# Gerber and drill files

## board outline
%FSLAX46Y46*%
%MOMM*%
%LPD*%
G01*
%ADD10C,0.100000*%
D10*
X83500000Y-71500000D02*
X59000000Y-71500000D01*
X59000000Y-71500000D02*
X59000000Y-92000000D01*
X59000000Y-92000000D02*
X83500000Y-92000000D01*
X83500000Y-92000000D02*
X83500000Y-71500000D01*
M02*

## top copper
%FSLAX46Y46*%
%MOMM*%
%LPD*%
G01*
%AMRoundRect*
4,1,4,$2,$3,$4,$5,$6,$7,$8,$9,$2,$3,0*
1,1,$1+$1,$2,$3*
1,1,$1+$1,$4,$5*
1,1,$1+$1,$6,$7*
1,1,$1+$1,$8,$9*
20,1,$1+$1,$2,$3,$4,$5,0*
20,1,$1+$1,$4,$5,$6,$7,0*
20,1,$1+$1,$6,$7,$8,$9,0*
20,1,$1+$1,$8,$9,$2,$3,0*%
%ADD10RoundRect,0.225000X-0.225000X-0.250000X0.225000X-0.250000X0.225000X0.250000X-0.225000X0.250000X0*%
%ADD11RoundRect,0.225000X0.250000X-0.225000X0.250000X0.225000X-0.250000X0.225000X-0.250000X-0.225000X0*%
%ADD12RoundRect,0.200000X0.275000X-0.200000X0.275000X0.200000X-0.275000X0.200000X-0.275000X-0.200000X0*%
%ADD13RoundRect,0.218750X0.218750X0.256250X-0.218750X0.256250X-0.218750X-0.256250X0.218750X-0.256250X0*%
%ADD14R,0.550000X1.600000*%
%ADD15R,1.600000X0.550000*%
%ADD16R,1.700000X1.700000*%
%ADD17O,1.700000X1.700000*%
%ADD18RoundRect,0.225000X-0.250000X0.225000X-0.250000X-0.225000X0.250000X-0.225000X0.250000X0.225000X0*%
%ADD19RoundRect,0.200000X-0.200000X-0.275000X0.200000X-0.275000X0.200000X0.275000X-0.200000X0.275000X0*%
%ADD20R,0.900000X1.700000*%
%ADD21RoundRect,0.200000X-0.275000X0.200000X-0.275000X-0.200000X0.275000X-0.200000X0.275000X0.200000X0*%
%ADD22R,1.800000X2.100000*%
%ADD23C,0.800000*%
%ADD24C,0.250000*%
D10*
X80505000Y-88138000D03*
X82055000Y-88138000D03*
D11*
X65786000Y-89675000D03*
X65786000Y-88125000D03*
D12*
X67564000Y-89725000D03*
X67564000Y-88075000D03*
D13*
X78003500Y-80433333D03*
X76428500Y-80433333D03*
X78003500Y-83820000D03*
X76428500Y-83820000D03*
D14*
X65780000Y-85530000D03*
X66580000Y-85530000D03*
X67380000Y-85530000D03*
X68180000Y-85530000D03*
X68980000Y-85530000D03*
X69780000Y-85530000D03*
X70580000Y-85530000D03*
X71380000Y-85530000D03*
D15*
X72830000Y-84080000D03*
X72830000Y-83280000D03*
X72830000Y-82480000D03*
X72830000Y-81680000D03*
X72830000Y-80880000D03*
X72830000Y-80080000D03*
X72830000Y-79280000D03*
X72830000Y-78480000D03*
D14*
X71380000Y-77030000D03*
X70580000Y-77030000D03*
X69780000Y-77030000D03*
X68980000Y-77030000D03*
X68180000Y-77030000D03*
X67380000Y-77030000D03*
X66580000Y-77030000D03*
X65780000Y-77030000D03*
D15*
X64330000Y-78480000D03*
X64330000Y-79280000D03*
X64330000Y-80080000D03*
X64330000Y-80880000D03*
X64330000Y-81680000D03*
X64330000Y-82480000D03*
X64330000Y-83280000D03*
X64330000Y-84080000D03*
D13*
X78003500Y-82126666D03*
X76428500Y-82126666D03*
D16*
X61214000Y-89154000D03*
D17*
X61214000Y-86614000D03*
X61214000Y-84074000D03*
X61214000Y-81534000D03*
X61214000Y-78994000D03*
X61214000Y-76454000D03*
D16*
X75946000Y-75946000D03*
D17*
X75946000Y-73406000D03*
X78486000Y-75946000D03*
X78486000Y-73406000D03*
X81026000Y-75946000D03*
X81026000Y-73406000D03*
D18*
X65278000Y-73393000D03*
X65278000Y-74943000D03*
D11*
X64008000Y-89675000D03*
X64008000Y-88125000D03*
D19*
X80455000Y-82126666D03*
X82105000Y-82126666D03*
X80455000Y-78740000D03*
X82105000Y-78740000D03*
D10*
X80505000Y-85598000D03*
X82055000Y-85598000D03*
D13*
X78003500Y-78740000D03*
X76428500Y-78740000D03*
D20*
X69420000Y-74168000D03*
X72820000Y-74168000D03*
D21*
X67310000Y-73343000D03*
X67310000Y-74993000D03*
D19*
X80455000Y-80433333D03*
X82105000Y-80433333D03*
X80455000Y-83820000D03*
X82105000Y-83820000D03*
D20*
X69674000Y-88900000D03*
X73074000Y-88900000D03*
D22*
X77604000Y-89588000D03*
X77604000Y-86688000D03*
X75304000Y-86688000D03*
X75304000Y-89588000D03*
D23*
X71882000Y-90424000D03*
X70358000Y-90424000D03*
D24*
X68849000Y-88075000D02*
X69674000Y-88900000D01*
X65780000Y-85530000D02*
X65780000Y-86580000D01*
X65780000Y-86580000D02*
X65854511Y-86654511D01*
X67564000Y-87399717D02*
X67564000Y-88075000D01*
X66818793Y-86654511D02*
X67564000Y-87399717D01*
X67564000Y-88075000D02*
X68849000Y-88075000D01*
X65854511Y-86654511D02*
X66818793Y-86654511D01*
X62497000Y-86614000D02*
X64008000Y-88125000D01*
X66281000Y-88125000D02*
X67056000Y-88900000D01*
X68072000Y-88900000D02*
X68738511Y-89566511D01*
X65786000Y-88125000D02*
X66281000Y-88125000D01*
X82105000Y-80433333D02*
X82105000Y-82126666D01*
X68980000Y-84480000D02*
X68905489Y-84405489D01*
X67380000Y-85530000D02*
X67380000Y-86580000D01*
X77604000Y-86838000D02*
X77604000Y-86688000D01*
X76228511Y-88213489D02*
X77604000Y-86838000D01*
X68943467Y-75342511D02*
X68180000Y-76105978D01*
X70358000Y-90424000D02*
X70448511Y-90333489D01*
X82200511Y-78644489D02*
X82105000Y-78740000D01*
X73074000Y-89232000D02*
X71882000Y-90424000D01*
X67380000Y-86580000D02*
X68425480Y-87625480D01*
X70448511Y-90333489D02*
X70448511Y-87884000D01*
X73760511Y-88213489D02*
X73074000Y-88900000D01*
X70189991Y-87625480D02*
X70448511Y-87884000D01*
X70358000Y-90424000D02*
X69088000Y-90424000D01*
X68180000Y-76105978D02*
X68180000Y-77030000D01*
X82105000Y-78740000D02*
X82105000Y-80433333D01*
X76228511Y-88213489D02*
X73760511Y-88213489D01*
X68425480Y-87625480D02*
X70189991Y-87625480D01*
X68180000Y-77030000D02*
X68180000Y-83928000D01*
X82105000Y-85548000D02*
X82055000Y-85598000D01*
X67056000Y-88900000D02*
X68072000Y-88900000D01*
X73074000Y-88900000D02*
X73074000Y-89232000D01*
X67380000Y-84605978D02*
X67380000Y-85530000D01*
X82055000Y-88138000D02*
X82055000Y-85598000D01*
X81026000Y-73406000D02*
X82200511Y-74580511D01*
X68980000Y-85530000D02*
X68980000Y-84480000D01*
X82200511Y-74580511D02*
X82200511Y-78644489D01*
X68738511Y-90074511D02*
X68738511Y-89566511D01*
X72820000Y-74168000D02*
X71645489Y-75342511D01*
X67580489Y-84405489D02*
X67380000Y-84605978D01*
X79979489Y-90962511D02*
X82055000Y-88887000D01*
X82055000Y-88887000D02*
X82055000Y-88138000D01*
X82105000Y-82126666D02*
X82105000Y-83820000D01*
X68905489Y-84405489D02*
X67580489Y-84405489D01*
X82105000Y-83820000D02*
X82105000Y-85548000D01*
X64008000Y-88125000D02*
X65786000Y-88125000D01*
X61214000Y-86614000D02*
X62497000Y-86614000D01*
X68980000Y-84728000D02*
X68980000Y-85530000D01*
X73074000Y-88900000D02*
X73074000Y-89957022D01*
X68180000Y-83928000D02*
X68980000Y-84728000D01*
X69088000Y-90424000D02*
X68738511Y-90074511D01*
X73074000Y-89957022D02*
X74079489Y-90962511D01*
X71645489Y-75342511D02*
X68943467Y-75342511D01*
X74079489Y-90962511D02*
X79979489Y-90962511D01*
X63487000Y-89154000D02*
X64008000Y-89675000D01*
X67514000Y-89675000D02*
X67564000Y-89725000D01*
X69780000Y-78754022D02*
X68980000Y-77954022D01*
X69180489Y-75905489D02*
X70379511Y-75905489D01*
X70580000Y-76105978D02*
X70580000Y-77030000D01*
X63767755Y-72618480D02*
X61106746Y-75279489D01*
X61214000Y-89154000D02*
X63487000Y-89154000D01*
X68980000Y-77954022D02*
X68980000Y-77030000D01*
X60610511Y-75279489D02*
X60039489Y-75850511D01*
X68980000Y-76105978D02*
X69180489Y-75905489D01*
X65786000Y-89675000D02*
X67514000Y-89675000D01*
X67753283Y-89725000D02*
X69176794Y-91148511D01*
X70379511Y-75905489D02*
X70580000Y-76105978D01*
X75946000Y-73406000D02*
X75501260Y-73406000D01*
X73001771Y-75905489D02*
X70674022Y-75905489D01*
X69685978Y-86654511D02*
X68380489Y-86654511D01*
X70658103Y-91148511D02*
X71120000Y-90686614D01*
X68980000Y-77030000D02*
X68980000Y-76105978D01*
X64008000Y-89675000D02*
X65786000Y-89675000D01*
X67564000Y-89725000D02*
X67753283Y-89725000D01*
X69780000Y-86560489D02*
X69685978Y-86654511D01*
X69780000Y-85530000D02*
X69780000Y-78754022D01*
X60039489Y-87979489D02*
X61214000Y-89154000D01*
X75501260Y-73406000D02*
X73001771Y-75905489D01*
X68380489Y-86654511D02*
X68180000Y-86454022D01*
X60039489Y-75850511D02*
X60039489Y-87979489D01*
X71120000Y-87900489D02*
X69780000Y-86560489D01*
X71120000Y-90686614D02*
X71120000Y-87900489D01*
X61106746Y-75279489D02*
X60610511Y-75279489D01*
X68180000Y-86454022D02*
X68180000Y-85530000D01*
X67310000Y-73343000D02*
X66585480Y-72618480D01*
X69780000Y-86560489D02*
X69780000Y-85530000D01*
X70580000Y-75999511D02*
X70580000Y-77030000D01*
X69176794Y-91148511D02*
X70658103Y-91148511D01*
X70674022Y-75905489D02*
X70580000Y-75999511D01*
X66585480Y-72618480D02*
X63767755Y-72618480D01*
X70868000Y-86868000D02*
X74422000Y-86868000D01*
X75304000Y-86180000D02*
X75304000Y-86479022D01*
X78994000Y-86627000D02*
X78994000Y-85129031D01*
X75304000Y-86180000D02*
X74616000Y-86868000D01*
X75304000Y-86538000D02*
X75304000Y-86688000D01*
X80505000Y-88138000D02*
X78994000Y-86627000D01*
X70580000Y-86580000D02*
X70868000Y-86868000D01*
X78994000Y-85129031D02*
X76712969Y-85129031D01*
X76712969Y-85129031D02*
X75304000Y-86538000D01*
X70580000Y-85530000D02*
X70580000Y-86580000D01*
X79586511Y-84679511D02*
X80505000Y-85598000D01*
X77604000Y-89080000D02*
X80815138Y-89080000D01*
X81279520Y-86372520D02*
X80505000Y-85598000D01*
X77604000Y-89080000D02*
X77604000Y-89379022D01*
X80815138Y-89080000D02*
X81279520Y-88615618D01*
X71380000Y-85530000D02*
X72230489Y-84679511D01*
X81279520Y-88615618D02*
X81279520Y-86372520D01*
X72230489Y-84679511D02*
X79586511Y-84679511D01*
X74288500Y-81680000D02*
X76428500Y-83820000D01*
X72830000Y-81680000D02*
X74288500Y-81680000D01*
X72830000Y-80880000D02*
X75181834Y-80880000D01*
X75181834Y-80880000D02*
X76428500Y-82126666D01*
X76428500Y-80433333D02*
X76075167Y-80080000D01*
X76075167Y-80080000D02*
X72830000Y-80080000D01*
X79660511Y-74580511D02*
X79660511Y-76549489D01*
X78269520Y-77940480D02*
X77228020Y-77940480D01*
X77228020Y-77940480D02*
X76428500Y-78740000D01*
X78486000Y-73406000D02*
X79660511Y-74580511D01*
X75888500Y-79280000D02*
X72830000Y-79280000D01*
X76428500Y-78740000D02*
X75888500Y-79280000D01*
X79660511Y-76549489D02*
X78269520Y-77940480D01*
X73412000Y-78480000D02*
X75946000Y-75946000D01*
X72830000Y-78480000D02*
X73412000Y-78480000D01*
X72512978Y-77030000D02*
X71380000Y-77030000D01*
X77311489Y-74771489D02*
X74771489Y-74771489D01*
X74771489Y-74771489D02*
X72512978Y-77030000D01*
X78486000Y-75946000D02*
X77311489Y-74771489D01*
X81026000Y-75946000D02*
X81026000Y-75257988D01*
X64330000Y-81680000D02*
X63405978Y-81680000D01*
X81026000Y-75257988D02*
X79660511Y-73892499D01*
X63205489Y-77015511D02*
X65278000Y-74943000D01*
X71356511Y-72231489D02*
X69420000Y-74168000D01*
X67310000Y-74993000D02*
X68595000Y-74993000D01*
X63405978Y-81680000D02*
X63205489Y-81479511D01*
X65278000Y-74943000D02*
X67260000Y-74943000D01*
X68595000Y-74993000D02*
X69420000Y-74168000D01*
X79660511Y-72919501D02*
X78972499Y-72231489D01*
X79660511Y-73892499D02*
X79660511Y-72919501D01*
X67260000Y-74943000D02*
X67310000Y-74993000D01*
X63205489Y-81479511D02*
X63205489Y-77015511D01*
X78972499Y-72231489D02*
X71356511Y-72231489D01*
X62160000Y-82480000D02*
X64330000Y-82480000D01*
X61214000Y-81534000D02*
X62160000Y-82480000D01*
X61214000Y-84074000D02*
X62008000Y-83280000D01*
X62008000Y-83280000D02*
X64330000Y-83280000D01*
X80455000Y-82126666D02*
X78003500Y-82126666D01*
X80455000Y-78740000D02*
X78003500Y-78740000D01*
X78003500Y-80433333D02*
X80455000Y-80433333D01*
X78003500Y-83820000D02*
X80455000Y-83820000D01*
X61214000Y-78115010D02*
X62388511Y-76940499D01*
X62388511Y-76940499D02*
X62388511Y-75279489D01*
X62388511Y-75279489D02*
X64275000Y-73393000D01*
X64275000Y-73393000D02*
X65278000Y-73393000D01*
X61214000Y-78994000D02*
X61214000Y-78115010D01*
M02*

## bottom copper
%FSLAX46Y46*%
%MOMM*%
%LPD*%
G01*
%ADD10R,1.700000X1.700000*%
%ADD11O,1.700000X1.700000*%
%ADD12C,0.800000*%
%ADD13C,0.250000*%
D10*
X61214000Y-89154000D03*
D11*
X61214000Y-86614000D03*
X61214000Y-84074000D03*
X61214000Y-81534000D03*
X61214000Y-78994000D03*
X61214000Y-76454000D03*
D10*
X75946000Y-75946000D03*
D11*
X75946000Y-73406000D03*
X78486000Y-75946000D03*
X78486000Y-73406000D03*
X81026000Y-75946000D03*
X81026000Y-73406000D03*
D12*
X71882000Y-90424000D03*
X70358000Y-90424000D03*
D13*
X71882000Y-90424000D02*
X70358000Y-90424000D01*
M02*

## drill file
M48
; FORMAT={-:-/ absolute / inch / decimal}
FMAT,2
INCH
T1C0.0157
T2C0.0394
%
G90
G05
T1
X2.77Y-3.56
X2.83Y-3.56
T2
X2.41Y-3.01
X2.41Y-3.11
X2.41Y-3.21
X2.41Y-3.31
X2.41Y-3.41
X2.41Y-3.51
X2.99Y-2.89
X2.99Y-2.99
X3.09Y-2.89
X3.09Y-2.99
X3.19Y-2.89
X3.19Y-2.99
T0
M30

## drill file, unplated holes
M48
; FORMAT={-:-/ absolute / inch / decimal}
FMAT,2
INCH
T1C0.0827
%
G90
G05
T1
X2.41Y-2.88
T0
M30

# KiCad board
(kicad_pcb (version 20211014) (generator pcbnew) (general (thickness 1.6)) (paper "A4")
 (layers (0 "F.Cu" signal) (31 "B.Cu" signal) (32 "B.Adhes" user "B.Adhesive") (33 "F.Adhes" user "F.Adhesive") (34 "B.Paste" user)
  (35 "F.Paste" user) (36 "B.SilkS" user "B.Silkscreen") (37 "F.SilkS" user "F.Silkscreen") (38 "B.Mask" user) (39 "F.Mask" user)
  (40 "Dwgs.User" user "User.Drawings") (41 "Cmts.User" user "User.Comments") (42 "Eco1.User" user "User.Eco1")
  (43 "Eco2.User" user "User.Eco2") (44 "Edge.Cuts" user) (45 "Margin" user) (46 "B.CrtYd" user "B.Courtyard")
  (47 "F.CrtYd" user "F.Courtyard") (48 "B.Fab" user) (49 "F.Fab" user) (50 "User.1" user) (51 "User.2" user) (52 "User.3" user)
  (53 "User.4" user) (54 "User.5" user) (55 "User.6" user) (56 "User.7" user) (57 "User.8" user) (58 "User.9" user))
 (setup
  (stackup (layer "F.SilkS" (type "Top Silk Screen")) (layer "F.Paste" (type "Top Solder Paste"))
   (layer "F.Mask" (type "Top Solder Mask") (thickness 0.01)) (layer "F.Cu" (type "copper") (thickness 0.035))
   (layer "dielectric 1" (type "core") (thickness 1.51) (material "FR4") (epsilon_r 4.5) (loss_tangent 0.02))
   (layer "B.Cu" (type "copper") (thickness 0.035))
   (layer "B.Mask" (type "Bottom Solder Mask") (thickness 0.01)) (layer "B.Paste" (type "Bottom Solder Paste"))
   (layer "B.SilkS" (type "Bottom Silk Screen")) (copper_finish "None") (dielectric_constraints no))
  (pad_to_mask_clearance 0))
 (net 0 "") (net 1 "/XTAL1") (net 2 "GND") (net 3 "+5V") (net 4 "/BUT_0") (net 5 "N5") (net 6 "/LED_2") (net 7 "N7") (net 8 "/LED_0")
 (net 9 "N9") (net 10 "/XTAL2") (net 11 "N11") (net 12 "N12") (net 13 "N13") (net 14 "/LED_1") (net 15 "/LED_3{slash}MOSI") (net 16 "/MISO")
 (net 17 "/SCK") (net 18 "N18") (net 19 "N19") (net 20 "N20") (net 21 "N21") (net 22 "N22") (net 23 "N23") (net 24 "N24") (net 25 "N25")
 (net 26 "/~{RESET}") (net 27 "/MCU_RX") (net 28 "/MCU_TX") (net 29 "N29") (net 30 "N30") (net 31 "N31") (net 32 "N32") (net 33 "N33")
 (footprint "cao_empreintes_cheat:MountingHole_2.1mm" (layer "F.Cu") (at 61.214 73.152)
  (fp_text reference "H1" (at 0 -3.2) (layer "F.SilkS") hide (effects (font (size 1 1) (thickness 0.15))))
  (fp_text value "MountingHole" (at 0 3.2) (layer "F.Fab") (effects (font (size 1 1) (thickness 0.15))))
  (pad "" np_thru_hole circle (at 0 0) (size 2.1 2.1) (drill 2.1) (layers *.Cu *.Mask)))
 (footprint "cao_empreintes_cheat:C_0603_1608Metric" (layer "F.Cu") (at 81.28 88.138)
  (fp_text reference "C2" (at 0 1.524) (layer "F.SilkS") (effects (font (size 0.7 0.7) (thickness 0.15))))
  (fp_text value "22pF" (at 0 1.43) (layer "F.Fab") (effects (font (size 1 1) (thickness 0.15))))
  (pad "1" smd roundrect (at -0.775 0) (size 0.9 0.95) (layers "F.Cu" "F.Paste" "F.Mask") (roundrect_rratio 0.25) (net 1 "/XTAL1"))
  (pad "2" smd roundrect (at 0.775 0) (size 0.9 0.95) (layers "F.Cu" "F.Paste" "F.Mask") (roundrect_rratio 0.25) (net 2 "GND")))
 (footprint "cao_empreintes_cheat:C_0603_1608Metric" (layer "F.Cu") (at 65.786 88.9 90)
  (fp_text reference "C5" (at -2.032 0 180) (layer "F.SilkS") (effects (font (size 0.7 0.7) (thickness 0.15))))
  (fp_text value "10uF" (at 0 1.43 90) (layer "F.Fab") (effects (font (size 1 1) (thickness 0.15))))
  (pad "1" smd roundrect (at -0.775 0 90) (size 0.9 0.95) (layers "F.Cu" "F.Paste" "F.Mask") (roundrect_rratio 0.25) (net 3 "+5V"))
  (pad "2" smd roundrect (at 0.775 0 90) (size 0.9 0.95) (layers "F.Cu" "F.Paste" "F.Mask") (roundrect_rratio 0.25) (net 2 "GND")))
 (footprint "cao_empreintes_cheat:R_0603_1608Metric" (layer "F.Cu") (at 67.564 88.9 90)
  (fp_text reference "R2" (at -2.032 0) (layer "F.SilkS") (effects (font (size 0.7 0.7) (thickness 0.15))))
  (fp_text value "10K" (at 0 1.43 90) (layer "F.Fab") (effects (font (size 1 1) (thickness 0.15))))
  (pad "1" smd roundrect (at -0.825 0 90) (size 0.8 0.95) (layers "F.Cu" "F.Paste" "F.Mask") (roundrect_rratio 0.25) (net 3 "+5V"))
  (pad "2" smd roundrect (at 0.825 0 90) (size 0.8 0.95) (layers "F.Cu" "F.Paste" "F.Mask") (roundrect_rratio 0.25) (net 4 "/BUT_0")))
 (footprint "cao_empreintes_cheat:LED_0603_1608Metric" (layer "F.Cu") (at 77.216 80.433333 180)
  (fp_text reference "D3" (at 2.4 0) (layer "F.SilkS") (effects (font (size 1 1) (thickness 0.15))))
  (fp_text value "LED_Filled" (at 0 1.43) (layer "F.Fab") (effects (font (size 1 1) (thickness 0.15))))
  (pad "1" smd roundrect (at -0.7875 0 180) (size 0.875 0.95) (layers "F.Cu" "F.Paste" "F.Mask") (roundrect_rratio 0.25) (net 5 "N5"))
  (pad "2" smd roundrect (at 0.7875 0 180) (size 0.875 0.95) (layers "F.Cu" "F.Paste" "F.Mask") (roundrect_rratio 0.25) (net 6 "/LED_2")))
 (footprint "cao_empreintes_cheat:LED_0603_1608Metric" (layer "F.Cu") (at 77.216 83.82 180)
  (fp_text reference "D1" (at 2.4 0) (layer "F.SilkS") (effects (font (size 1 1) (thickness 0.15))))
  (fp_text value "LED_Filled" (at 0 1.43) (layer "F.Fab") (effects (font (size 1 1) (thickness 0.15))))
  (pad "1" smd roundrect (at -0.7875 0 180) (size 0.875 0.95) (layers "F.Cu" "F.Paste" "F.Mask") (roundrect_rratio 0.25) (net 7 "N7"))
  (pad "2" smd roundrect (at 0.7875 0 180) (size 0.875 0.95) (layers "F.Cu" "F.Paste" "F.Mask") (roundrect_rratio 0.25) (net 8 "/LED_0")))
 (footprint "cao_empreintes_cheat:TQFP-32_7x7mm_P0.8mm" (layer "F.Cu") (at 68.58 81.28 90)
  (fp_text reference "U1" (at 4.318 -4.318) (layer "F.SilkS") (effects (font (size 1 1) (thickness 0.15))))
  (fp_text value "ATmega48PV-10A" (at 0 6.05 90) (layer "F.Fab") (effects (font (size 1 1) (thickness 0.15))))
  (pad "1" smd rect (at -4.25 -2.8 90) (size 1.6 0.55) (layers "F.Cu" "F.Paste" "F.Mask") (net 4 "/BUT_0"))
  (pad "2" smd rect (at -4.25 -2 90) (size 1.6 0.55) (layers "F.Cu" "F.Paste" "F.Mask") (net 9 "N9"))
  (pad "3" smd rect (at -4.25 -1.2 90) (size 1.6 0.55) (layers "F.Cu" "F.Paste" "F.Mask") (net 2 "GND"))
  (pad "4" smd rect (at -4.25 -0.4 90) (size 1.6 0.55) (layers "F.Cu" "F.Paste" "F.Mask") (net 3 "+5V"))
  (pad "5" smd rect (at -4.25 0.4 90) (size 1.6 0.55) (layers "F.Cu" "F.Paste" "F.Mask") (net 2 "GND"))
  (pad "6" smd rect (at -4.25 1.2 90) (size 1.6 0.55) (layers "F.Cu" "F.Paste" "F.Mask") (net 3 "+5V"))
  (pad "7" smd rect (at -4.25 2 90) (size 1.6 0.55) (layers "F.Cu" "F.Paste" "F.Mask") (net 1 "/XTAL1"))
  (pad "8" smd rect (at -4.25 2.8 90) (size 1.6 0.55) (layers "F.Cu" "F.Paste" "F.Mask") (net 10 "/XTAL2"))
  (pad "9" smd rect (at -2.8 4.25 180) (size 1.6 0.55) (layers "F.Cu" "F.Paste" "F.Mask") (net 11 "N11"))
  (pad "10" smd rect (at -2 4.25 180) (size 1.6 0.55) (layers "F.Cu" "F.Paste" "F.Mask") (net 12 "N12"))
  (pad "11" smd rect (at -1.2 4.25 180) (size 1.6 0.55) (layers "F.Cu" "F.Paste" "F.Mask") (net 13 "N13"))
  (pad "12" smd rect (at -0.4 4.25 180) (size 1.6 0.55) (layers "F.Cu" "F.Paste" "F.Mask") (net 8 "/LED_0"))
  (pad "13" smd rect (at 0.4 4.25 180) (size 1.6 0.55) (layers "F.Cu" "F.Paste" "F.Mask") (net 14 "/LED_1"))
  (pad "14" smd rect (at 1.2 4.25 180) (size 1.6 0.55) (layers "F.Cu" "F.Paste" "F.Mask") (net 6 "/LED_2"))
  (pad "15" smd rect (at 2 4.25 180) (size 1.6 0.55) (layers "F.Cu" "F.Paste" "F.Mask") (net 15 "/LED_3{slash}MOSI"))
  (pad "16" smd rect (at 2.8 4.25 180) (size 1.6 0.55) (layers "F.Cu" "F.Paste" "F.Mask") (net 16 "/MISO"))
  (pad "17" smd rect (at 4.25 2.8 90) (size 1.6 0.55) (layers "F.Cu" "F.Paste" "F.Mask") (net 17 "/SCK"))
  (pad "18" smd rect (at 4.25 2 90) (size 1.6 0.55) (layers "F.Cu" "F.Paste" "F.Mask") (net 3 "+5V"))
  (pad "19" smd rect (at 4.25 1.2 90) (size 1.6 0.55) (layers "F.Cu" "F.Paste" "F.Mask") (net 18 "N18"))
  (pad "20" smd rect (at 4.25 0.4 90) (size 1.6 0.55) (layers "F.Cu" "F.Paste" "F.Mask") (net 3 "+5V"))
  (pad "21" smd rect (at 4.25 -0.4 90) (size 1.6 0.55) (layers "F.Cu" "F.Paste" "F.Mask") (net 2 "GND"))
  (pad "22" smd rect (at 4.25 -1.2 90) (size 1.6 0.55) (layers "F.Cu" "F.Paste" "F.Mask") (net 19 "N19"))
  (pad "23" smd rect (at 4.25 -2 90) (size 1.6 0.55) (layers "F.Cu" "F.Paste" "F.Mask") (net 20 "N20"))
  (pad "24" smd rect (at 4.25 -2.8 90) (size 1.6 0.55) (layers "F.Cu" "F.Paste" "F.Mask") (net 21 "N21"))
  (pad "25" smd rect (at 2.8 -4.25 180) (size 1.6 0.55) (layers "F.Cu" "F.Paste" "F.Mask") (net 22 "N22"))
  (pad "26" smd rect (at 2 -4.25 180) (size 1.6 0.55) (layers "F.Cu" "F.Paste" "F.Mask") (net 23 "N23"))
  (pad "27" smd rect (at 1.2 -4.25 180) (size 1.6 0.55) (layers "F.Cu" "F.Paste" "F.Mask") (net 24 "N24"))
  (pad "28" smd rect (at 0.4 -4.25 180) (size 1.6 0.55) (layers "F.Cu" "F.Paste" "F.Mask") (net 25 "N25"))
  (pad "29" smd rect (at -0.4 -4.25 180) (size 1.6 0.55) (layers "F.Cu" "F.Paste" "F.Mask") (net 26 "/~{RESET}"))
  (pad "30" smd rect (at -1.2 -4.25 180) (size 1.6 0.55) (layers "F.Cu" "F.Paste" "F.Mask") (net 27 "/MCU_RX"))
  (pad "31" smd rect (at -2 -4.25 180) (size 1.6 0.55) (layers "F.Cu" "F.Paste" "F.Mask") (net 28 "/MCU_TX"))
  (pad "32" smd rect (at -2.8 -4.25 180) (size 1.6 0.55) (layers "F.Cu" "F.Paste" "F.Mask") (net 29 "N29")))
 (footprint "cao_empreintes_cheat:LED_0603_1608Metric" (layer "F.Cu") (at 77.216 82.126666 180)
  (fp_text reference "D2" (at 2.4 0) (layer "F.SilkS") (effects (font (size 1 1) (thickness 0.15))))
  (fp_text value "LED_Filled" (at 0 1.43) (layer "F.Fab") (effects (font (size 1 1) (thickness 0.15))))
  (pad "1" smd roundrect (at -0.7875 0 180) (size 0.875 0.95) (layers "F.Cu" "F.Paste" "F.Mask") (roundrect_rratio 0.25) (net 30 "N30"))
  (pad "2" smd roundrect (at 0.7875 0 180) (size 0.875 0.95) (layers "F.Cu" "F.Paste" "F.Mask") (roundrect_rratio 0.25) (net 14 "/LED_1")))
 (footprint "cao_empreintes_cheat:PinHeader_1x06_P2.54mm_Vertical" (layer "F.Cu") (at 61.214 89.154 180)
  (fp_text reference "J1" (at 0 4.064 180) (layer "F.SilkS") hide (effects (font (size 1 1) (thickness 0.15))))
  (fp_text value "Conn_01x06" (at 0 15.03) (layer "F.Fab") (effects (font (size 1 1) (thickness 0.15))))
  (pad "1" thru_hole rect (at 0 0 180) (size 1.7 1.7) (drill 1) (layers *.Cu *.Mask) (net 3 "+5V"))
  (pad "2" thru_hole oval (at 0 2.54 180) (size 1.7 1.7) (drill 1) (layers *.Cu *.Mask) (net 2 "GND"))
  (pad "3" thru_hole oval (at 0 5.08 180) (size 1.7 1.7) (drill 1) (layers *.Cu *.Mask) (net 28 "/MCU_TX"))
  (pad "4" thru_hole oval (at 0 7.62 180) (size 1.7 1.7) (drill 1) (layers *.Cu *.Mask) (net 27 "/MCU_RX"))
  (pad "5" thru_hole oval (at 0 10.16 180) (size 1.7 1.7) (drill 1) (layers *.Cu *.Mask) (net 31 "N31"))
  (pad "6" thru_hole oval (at 0 12.7 180) (size 1.7 1.7) (drill 1) (layers *.Cu *.Mask) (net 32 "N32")))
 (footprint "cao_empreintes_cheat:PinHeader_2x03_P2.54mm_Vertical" (layer "F.Cu") (at 75.946 75.946 90)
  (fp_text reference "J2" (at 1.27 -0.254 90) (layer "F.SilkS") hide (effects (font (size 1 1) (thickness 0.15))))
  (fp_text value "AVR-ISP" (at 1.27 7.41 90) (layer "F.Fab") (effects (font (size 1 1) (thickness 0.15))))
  (pad "1" thru_hole rect (at 0 0 90) (size 1.7 1.7) (drill 1) (layers *.Cu *.Mask) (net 16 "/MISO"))
  (pad "2" thru_hole oval (at 2.54 0 90) (size 1.7 1.7) (drill 1) (layers *.Cu *.Mask) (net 3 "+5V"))
  (pad "3" thru_hole oval (at 0 2.54 90) (size 1.7 1.7) (drill 1) (layers *.Cu *.Mask) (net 17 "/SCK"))
  (pad "4" thru_hole oval (at 2.54 2.54 90) (size 1.7 1.7) (drill 1) (layers *.Cu *.Mask) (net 15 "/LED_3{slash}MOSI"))
  (pad "5" thru_hole oval (at 0 5.08 90) (size 1.7 1.7) (drill 1) (layers *.Cu *.Mask) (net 26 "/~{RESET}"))
  (pad "6" thru_hole oval (at 2.54 5.08 90) (size 1.7 1.7) (drill 1) (layers *.Cu *.Mask) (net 2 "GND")))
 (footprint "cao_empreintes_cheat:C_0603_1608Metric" (layer "F.Cu") (at 65.278 74.168 -90)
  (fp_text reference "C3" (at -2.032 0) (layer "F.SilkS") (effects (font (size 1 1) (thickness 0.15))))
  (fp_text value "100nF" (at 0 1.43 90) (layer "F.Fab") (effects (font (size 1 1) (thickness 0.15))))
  (pad "1" smd roundrect (at -0.775 0 270) (size 0.9 0.95) (layers "F.Cu" "F.Paste" "F.Mask") (roundrect_rratio 0.25) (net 31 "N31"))
  (pad "2" smd roundrect (at 0.775 0 270) (size 0.9 0.95) (layers "F.Cu" "F.Paste" "F.Mask") (roundrect_rratio 0.25) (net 26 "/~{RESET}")))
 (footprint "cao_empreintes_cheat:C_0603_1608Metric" (layer "F.Cu") (at 64.008 88.9 90)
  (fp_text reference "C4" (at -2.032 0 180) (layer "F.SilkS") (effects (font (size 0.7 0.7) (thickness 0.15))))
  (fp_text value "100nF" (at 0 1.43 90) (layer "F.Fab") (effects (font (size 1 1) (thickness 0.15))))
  (pad "1" smd roundrect (at -0.775 0 90) (size 0.9 0.95) (layers "F.Cu" "F.Paste" "F.Mask") (roundrect_rratio 0.25) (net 3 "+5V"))
  (pad "2" smd roundrect (at 0.775 0 90) (size 0.9 0.95) (layers "F.Cu" "F.Paste" "F.Mask") (roundrect_rratio 0.25) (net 2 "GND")))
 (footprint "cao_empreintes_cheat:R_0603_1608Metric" (layer "F.Cu") (at 81.28 82.126666)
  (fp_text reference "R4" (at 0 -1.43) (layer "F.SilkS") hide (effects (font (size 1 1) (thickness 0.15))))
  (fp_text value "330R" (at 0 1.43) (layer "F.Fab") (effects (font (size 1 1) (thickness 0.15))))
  (pad "1" smd roundrect (at -0.825 0) (size 0.8 0.95) (layers "F.Cu" "F.Paste" "F.Mask") (roundrect_rratio 0.25) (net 30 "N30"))
  (pad "2" smd roundrect (at 0.825 0) (size 0.8 0.95) (layers "F.Cu" "F.Paste" "F.Mask") (roundrect_rratio 0.25) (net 2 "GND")))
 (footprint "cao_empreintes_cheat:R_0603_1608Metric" (layer "F.Cu") (at 81.28 78.74)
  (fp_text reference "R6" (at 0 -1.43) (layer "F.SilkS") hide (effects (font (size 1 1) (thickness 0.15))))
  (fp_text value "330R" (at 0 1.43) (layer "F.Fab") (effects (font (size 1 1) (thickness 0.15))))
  (pad "1" smd roundrect (at -0.825 0) (size 0.8 0.95) (layers "F.Cu" "F.Paste" "F.Mask") (roundrect_rratio 0.25) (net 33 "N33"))
  (pad "2" smd roundrect (at 0.825 0) (size 0.8 0.95) (layers "F.Cu" "F.Paste" "F.Mask") (roundrect_rratio 0.25) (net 2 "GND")))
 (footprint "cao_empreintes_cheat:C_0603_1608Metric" (layer "F.Cu") (at 81.28 85.598)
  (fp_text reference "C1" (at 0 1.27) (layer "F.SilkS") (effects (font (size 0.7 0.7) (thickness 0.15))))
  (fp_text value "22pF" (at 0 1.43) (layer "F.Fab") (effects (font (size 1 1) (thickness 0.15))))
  (pad "1" smd roundrect (at -0.775 0) (size 0.9 0.95) (layers "F.Cu" "F.Paste" "F.Mask") (roundrect_rratio 0.25) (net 10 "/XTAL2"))
  (pad "2" smd roundrect (at 0.775 0) (size 0.9 0.95) (layers "F.Cu" "F.Paste" "F.Mask") (roundrect_rratio 0.25) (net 2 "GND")))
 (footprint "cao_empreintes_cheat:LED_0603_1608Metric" (layer "F.Cu") (at 77.216 78.74 180)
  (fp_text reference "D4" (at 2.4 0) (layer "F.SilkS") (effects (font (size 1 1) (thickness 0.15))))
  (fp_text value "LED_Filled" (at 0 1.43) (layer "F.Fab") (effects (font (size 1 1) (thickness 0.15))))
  (pad "1" smd roundrect (at -0.7875 0 180) (size 0.875 0.95) (layers "F.Cu" "F.Paste" "F.Mask") (roundrect_rratio 0.25) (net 33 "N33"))
  (pad "2" smd roundrect (at 0.7875 0 180) (size 0.875 0.95) (layers "F.Cu" "F.Paste" "F.Mask") (roundrect_rratio 0.25)
   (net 15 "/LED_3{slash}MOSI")))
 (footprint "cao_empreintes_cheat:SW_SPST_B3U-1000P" (layer "F.Cu") (at 71.12 74.168)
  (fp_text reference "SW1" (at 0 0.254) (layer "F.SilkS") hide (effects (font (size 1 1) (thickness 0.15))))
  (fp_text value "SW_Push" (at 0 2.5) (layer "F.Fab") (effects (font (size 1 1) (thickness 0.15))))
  (pad "1" smd rect (at -1.7 0) (size 0.9 1.7) (layers "F.Cu" "F.Paste" "F.Mask") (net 26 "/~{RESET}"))
  (pad "2" smd rect (at 1.7 0) (size 0.9 1.7) (layers "F.Cu" "F.Paste" "F.Mask") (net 2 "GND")))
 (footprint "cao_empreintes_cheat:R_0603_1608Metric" (layer "F.Cu") (at 67.31 74.168 -90)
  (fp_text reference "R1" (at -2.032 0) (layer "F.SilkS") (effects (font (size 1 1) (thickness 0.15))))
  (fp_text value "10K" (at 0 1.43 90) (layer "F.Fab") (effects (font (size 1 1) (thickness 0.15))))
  (pad "1" smd roundrect (at -0.825 0 270) (size 0.8 0.95) (layers "F.Cu" "F.Paste" "F.Mask") (roundrect_rratio 0.25) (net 3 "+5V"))
  (pad "2" smd roundrect (at 0.825 0 270) (size 0.8 0.95) (layers "F.Cu" "F.Paste" "F.Mask") (roundrect_rratio 0.25) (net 26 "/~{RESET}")))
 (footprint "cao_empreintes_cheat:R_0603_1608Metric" (layer "F.Cu") (at 81.28 80.433333)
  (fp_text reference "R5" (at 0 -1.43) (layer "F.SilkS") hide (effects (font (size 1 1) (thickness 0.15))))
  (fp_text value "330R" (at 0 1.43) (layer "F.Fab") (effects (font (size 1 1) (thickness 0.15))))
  (pad "1" smd roundrect (at -0.825 0) (size 0.8 0.95) (layers "F.Cu" "F.Paste" "F.Mask") (roundrect_rratio 0.25) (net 5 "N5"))
  (pad "2" smd roundrect (at 0.825 0) (size 0.8 0.95) (layers "F.Cu" "F.Paste" "F.Mask") (roundrect_rratio 0.25) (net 2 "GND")))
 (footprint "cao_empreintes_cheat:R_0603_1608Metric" (layer "F.Cu") (at 81.28 83.82)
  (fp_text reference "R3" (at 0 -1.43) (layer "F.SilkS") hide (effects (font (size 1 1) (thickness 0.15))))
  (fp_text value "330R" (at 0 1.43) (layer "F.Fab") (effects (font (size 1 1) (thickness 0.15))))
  (pad "1" smd roundrect (at -0.825 0) (size 0.8 0.95) (layers "F.Cu" "F.Paste" "F.Mask") (roundrect_rratio 0.25) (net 7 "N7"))
  (pad "2" smd roundrect (at 0.825 0) (size 0.8 0.95) (layers "F.Cu" "F.Paste" "F.Mask") (roundrect_rratio 0.25) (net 2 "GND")))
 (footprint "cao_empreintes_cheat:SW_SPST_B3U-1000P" (layer "F.Cu") (at 71.374 88.9)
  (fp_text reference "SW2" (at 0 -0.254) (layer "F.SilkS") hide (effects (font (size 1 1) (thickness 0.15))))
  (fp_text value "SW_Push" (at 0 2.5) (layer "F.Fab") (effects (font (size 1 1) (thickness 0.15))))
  (pad "1" smd rect (at -1.7 0) (size 0.9 1.7) (layers "F.Cu" "F.Paste" "F.Mask") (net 4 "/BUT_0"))
  (pad "2" smd rect (at 1.7 0) (size 0.9 1.7) (layers "F.Cu" "F.Paste" "F.Mask") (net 2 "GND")))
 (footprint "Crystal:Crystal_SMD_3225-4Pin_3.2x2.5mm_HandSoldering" (layer "F.Cu") (at 76.454 88.138 90)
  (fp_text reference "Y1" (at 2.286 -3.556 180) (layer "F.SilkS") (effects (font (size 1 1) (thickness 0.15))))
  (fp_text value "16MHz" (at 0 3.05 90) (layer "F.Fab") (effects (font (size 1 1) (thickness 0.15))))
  (pad "1" smd rect locked (at -1.45 1.15 90) (size 2.1 1.8) (layers "F.Cu" "F.Paste" "F.Mask") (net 10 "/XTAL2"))
  (pad "2" smd rect locked (at 1.45 1.15 90) (size 2.1 1.8) (layers "F.Cu" "F.Paste" "F.Mask") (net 2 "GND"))
  (pad "3" smd rect locked (at 1.45 -1.15 90) (size 2.1 1.8) (layers "F.Cu" "F.Paste" "F.Mask") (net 1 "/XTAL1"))
  (pad "4" smd rect locked (at -1.45 -1.15 90) (size 2.1 1.8) (layers "F.Cu" "F.Paste" "F.Mask")))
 (gr_rect (start 83.5 71.5) (end 59 92) (layer "Edge.Cuts") (width 0.1) (fill none))
 (segment (start 68.849 88.075) (end 69.674 88.9) (width 0.25) (layer "F.Cu") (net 4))
 (segment (start 65.78 85.53) (end 65.78 86.58) (width 0.25) (layer "F.Cu") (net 4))
 (segment (start 65.78 86.58) (end 65.854511 86.654511) (width 0.25) (layer "F.Cu") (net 4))
 (segment (start 67.564 87.399717) (end 67.564 88.075) (width 0.25) (layer "F.Cu") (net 4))
 (segment (start 66.818793 86.654511) (end 67.564 87.399717) (width 0.25) (layer "F.Cu") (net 4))
 (segment (start 67.564 88.075) (end 68.849 88.075) (width 0.25) (layer "F.Cu") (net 4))
 (segment (start 65.854511 86.654511) (end 66.818793 86.654511) (width 0.25) (layer "F.Cu") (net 4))
 (segment (start 62.497 86.614) (end 64.008 88.125) (width 0.25) (layer "F.Cu") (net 2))
 (segment (start 66.281 88.125) (end 67.056 88.9) (width 0.25) (layer "F.Cu") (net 2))
 (segment (start 68.072 88.9) (end 68.738511 89.566511) (width 0.25) (layer "F.Cu") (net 2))
 (segment (start 65.786 88.125) (end 66.281 88.125) (width 0.25) (layer "F.Cu") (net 2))
 (segment (start 82.105 80.433333) (end 82.105 82.126666) (width 0.25) (layer "F.Cu") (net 2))
 (segment (start 68.98 84.48) (end 68.905489 84.405489) (width 0.25) (layer "F.Cu") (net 2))
 (segment (start 67.38 85.53) (end 67.38 86.58) (width 0.25) (layer "F.Cu") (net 2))
 (segment (start 77.604 86.838) (end 77.604 86.688) (width 0.25) (layer "F.Cu") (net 2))
 (segment (start 76.228511 88.213489) (end 77.604 86.838) (width 0.25) (layer "F.Cu") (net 2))
 (segment (start 68.943467 75.342511) (end 68.18 76.105978) (width 0.25) (layer "F.Cu") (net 2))
 (segment (start 70.358 90.424) (end 70.448511 90.333489) (width 0.25) (layer "F.Cu") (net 2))
 (segment (start 82.200511 78.644489) (end 82.105 78.74) (width 0.25) (layer "F.Cu") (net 2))
 (segment (start 73.074 89.232) (end 71.882 90.424) (width 0.25) (layer "F.Cu") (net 2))
 (segment (start 67.38 86.58) (end 68.42548 87.62548) (width 0.25) (layer "F.Cu") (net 2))
 (segment (start 70.448511 90.333489) (end 70.448511 87.884) (width 0.25) (layer "F.Cu") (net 2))
 (segment (start 73.760511 88.213489) (end 73.074 88.9) (width 0.25) (layer "F.Cu") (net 2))
 (segment (start 70.189991 87.62548) (end 70.448511 87.884) (width 0.25) (layer "F.Cu") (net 2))
 (segment (start 70.358 90.424) (end 69.088 90.424) (width 0.25) (layer "F.Cu") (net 2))
 (segment (start 68.18 76.105978) (end 68.18 77.03) (width 0.25) (layer "F.Cu") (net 2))
 (segment (start 82.105 78.74) (end 82.105 80.433333) (width 0.25) (layer "F.Cu") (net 2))
 (segment (start 76.228511 88.213489) (end 73.760511 88.213489) (width 0.25) (layer "F.Cu") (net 2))
 (segment (start 68.42548 87.62548) (end 70.189991 87.62548) (width 0.25) (layer "F.Cu") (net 2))
 (segment (start 68.18 77.03) (end 68.18 83.928) (width 0.25) (layer "F.Cu") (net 2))
 (segment (start 82.105 85.548) (end 82.055 85.598) (width 0.25) (layer "F.Cu") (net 2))
 (segment (start 67.056 88.9) (end 68.072 88.9) (width 0.25) (layer "F.Cu") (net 2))
 (segment (start 73.074 88.9) (end 73.074 89.232) (width 0.25) (layer "F.Cu") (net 2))
 (segment (start 67.38 84.605978) (end 67.38 85.53) (width 0.25) (layer "F.Cu") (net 2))
 (segment (start 82.055 88.138) (end 82.055 85.598) (width 0.25) (layer "F.Cu") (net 2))
 (segment (start 81.026 73.406) (end 82.200511 74.580511) (width 0.25) (layer "F.Cu") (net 2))
 (segment (start 68.98 85.53) (end 68.98 84.48) (width 0.25) (layer "F.Cu") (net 2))
 (segment (start 82.200511 74.580511) (end 82.200511 78.644489) (width 0.25) (layer "F.Cu") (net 2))
 (segment (start 68.738511 90.074511) (end 68.738511 89.566511) (width 0.25) (layer "F.Cu") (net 2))
 (segment (start 72.82 74.168) (end 71.645489 75.342511) (width 0.25) (layer "F.Cu") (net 2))
 (segment (start 67.580489 84.405489) (end 67.38 84.605978) (width 0.25) (layer "F.Cu") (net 2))
 (segment (start 79.979489 90.962511) (end 82.055 88.887) (width 0.25) (layer "F.Cu") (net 2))
 (segment (start 82.055 88.887) (end 82.055 88.138) (width 0.25) (layer "F.Cu") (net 2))
 (segment (start 82.105 82.126666) (end 82.105 83.82) (width 0.25) (layer "F.Cu") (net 2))
 (segment (start 68.905489 84.405489) (end 67.580489 84.405489) (width 0.25) (layer "F.Cu") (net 2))
 (segment (start 82.105 83.82) (end 82.105 85.548) (width 0.25) (layer "F.Cu") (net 2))
 (segment (start 64.008 88.125) (end 65.786 88.125) (width 0.25) (layer "F.Cu") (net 2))
 (segment (start 61.214 86.614) (end 62.497 86.614) (width 0.25) (layer "F.Cu") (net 2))
 (segment (start 68.98 84.728) (end 68.98 85.53) (width 0.25) (layer "F.Cu") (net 2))
 (segment (start 73.074 88.9) (end 73.074 89.957022) (width 0.25) (layer "F.Cu") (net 2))
 (segment (start 68.18 83.928) (end 68.98 84.728) (width 0.25) (layer "F.Cu") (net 2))
 (segment (start 69.088 90.424) (end 68.738511 90.074511) (width 0.25) (layer "F.Cu") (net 2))
 (segment (start 73.074 89.957022) (end 74.079489 90.962511) (width 0.25) (layer "F.Cu") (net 2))
 (segment (start 71.645489 75.342511) (end 68.943467 75.342511) (width 0.25) (layer "F.Cu") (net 2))
 (segment (start 74.079489 90.962511) (end 79.979489 90.962511) (width 0.25) (layer "F.Cu") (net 2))
 (via (at 71.882 90.424) (size 0.8) (drill 0.4) (layers "F.Cu" "B.Cu") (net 2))
 (via (at 70.358 90.424) (size 0.8) (drill 0.4) (layers "F.Cu" "B.Cu") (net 2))
 (segment (start 71.882 90.424) (end 70.358 90.424) (width 0.25) (layer "B.Cu") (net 2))
 (segment (start 63.487 89.154) (end 64.008 89.675) (width 0.25) (layer "F.Cu") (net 3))
 (segment (start 67.514 89.675) (end 67.564 89.725) (width 0.25) (layer "F.Cu") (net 3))
 (segment (start 69.78 78.754022) (end 68.98 77.954022) (width 0.25) (layer "F.Cu") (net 3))
 (segment (start 69.180489 75.905489) (end 70.379511 75.905489) (width 0.25) (layer "F.Cu") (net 3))
 (segment (start 70.58 76.105978) (end 70.58 77.03) (width 0.25) (layer "F.Cu") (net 3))
 (segment (start 63.767755 72.61848) (end 61.106746 75.279489) (width 0.25) (layer "F.Cu") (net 3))
 (segment (start 61.214 89.154) (end 63.487 89.154) (width 0.25) (layer "F.Cu") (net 3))
 (segment (start 68.98 77.954022) (end 68.98 77.03) (width 0.25) (layer "F.Cu") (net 3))
 (segment (start 60.610511 75.279489) (end 60.039489 75.850511) (width 0.25) (layer "F.Cu") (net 3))
 (segment (start 68.98 76.105978) (end 69.180489 75.905489) (width 0.25) (layer "F.Cu") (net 3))
 (segment (start 65.786 89.675) (end 67.514 89.675) (width 0.25) (layer "F.Cu") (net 3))
 (segment (start 67.753283 89.725) (end 69.176794 91.148511) (width 0.25) (layer "F.Cu") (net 3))
 (segment (start 70.379511 75.905489) (end 70.58 76.105978) (width 0.25) (layer "F.Cu") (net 3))
 (segment (start 75.946 73.406) (end 75.50126 73.406) (width 0.25) (layer "F.Cu") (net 3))
 (segment (start 73.001771 75.905489) (end 70.674022 75.905489) (width 0.25) (layer "F.Cu") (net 3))
 (segment (start 69.685978 86.654511) (end 68.380489 86.654511) (width 0.25) (layer "F.Cu") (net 3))
 (segment (start 70.658103 91.148511) (end 71.12 90.686614) (width 0.25) (layer "F.Cu") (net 3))
 (segment (start 68.98 77.03) (end 68.98 76.105978) (width 0.25) (layer "F.Cu") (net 3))
 (segment (start 64.008 89.675) (end 65.786 89.675) (width 0.25) (layer "F.Cu") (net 3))
 (segment (start 67.564 89.725) (end 67.753283 89.725) (width 0.25) (layer "F.Cu") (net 3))
 (segment (start 69.78 86.560489) (end 69.685978 86.654511) (width 0.25) (layer "F.Cu") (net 3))
 (segment (start 69.78 85.53) (end 69.78 78.754022) (width 0.25) (layer "F.Cu") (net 3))
 (segment (start 60.039489 87.979489) (end 61.214 89.154) (width 0.25) (layer "F.Cu") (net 3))
 (segment (start 75.50126 73.406) (end 73.001771 75.905489) (width 0.25) (layer "F.Cu") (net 3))
 (segment (start 68.380489 86.654511) (end 68.18 86.454022) (width 0.25) (layer "F.Cu") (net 3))
 (segment (start 60.039489 75.850511) (end 60.039489 87.979489) (width 0.25) (layer "F.Cu") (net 3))
 (segment (start 71.12 87.900489) (end 69.78 86.560489) (width 0.25) (layer "F.Cu") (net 3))
 (segment (start 71.12 90.686614) (end 71.12 87.900489) (width 0.25) (layer "F.Cu") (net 3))
 (segment (start 61.106746 75.279489) (end 60.610511 75.279489) (width 0.25) (layer "F.Cu") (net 3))
 (segment (start 68.18 86.454022) (end 68.18 85.53) (width 0.25) (layer "F.Cu") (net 3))
 (segment (start 67.31 73.343) (end 66.58548 72.61848) (width 0.25) (layer "F.Cu") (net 3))
 (segment (start 69.78 86.560489) (end 69.78 85.53) (width 0.25) (layer "F.Cu") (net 3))
 (segment (start 70.58 75.999511) (end 70.58 77.03) (width 0.25) (layer "F.Cu") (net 3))
 (segment (start 69.176794 91.148511) (end 70.658103 91.148511) (width 0.25) (layer "F.Cu") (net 3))
 (segment (start 70.674022 75.905489) (end 70.58 75.999511) (width 0.25) (layer "F.Cu") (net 3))
 (segment (start 66.58548 72.61848) (end 63.767755 72.61848) (width 0.25) (layer "F.Cu") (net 3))
 (segment (start 70.868 86.868) (end 74.422 86.868) (width 0.25) (layer "F.Cu") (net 1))
 (segment (start 75.304 86.18) (end 75.304 86.479022) (width 0.25) (layer "F.Cu") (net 1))
 (segment (start 78.994 86.627) (end 78.994 85.129031) (width 0.25) (layer "F.Cu") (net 1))
 (segment (start 75.304 86.18) (end 74.616 86.868) (width 0.25) (layer "F.Cu") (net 1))
 (segment (start 75.304 86.538) (end 75.304 86.688) (width 0.25) (layer "F.Cu") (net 1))
 (segment (start 80.505 88.138) (end 78.994 86.627) (width 0.25) (layer "F.Cu") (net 1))
 (segment (start 70.58 86.58) (end 70.868 86.868) (width 0.25) (layer "F.Cu") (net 1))
 (segment (start 78.994 85.129031) (end 76.712969 85.129031) (width 0.25) (layer "F.Cu") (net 1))
 (segment (start 76.712969 85.129031) (end 75.304 86.538) (width 0.25) (layer "F.Cu") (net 1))
 (segment (start 70.58 85.53) (end 70.58 86.58) (width 0.25) (layer "F.Cu") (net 1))
 (segment (start 79.586511 84.679511) (end 80.505 85.598) (width 0.25) (layer "F.Cu") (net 10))
 (segment (start 77.604 89.08) (end 80.815138 89.08) (width 0.25) (layer "F.Cu") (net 10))
 (segment (start 81.27952 86.37252) (end 80.505 85.598) (width 0.25) (layer "F.Cu") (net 10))
 (segment (start 77.604 89.08) (end 77.604 89.379022) (width 0.25) (layer "F.Cu") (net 10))
 (segment (start 80.815138 89.08) (end 81.27952 88.615618) (width 0.25) (layer "F.Cu") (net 10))
 (segment (start 71.38 85.53) (end 72.230489 84.679511) (width 0.25) (layer "F.Cu") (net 10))
 (segment (start 81.27952 88.615618) (end 81.27952 86.37252) (width 0.25) (layer "F.Cu") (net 10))
 (segment (start 72.230489 84.679511) (end 79.586511 84.679511) (width 0.25) (layer "F.Cu") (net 10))
 (segment (start 74.2885 81.68) (end 76.4285 83.82) (width 0.25) (layer "F.Cu") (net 8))
 (segment (start 72.83 81.68) (end 74.2885 81.68) (width 0.25) (layer "F.Cu") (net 8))
 (segment (start 72.83 80.88) (end 75.181834 80.88) (width 0.25) (layer "F.Cu") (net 14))
 (segment (start 75.181834 80.88) (end 76.4285 82.126666) (width 0.25) (layer "F.Cu") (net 14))
 (segment (start 76.4285 80.433333) (end 76.075167 80.08) (width 0.25) (layer "F.Cu") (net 6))
 (segment (start 76.075167 80.08) (end 72.83 80.08) (width 0.25) (layer "F.Cu") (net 6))
 (segment (start 79.660511 74.580511) (end 79.660511 76.549489) (width 0.25) (layer "F.Cu") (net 15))
 (segment (start 78.26952 77.94048) (end 77.22802 77.94048) (width 0.25) (layer "F.Cu") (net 15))
 (segment (start 77.22802 77.94048) (end 76.4285 78.74) (width 0.25) (layer "F.Cu") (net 15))
 (segment (start 78.486 73.406) (end 79.660511 74.580511) (width 0.25) (layer "F.Cu") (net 15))
 (segment (start 75.8885 79.28) (end 72.83 79.28) (width 0.25) (layer "F.Cu") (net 15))
 (segment (start 76.4285 78.74) (end 75.8885 79.28) (width 0.25) (layer "F.Cu") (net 15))
 (segment (start 79.660511 76.549489) (end 78.26952 77.94048) (width 0.25) (layer "F.Cu") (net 15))
 (segment (start 73.412 78.48) (end 75.946 75.946) (width 0.25) (layer "F.Cu") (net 16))
 (segment (start 72.83 78.48) (end 73.412 78.48) (width 0.25) (layer "F.Cu") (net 16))
 (segment (start 72.512978 77.03) (end 71.38 77.03) (width 0.25) (layer "F.Cu") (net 17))
 (segment (start 77.311489 74.771489) (end 74.771489 74.771489) (width 0.25) (layer "F.Cu") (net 17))
 (segment (start 74.771489 74.771489) (end 72.512978 77.03) (width 0.25) (layer "F.Cu") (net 17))
 (segment (start 78.486 75.946) (end 77.311489 74.771489) (width 0.25) (layer "F.Cu") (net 17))
 (segment (start 81.026 75.946) (end 81.026 75.257988) (width 0.25) (layer "F.Cu") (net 26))
 (segment (start 64.33 81.68) (end 63.405978 81.68) (width 0.25) (layer "F.Cu") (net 26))
 (segment (start 81.026 75.257988) (end 79.660511 73.892499) (width 0.25) (layer "F.Cu") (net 26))
 (segment (start 63.205489 77.015511) (end 65.278 74.943) (width 0.25) (layer "F.Cu") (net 26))
 (segment (start 71.356511 72.231489) (end 69.42 74.168) (width 0.25) (layer "F.Cu") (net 26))
 (segment (start 67.31 74.993) (end 68.595 74.993) (width 0.25) (layer "F.Cu") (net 26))
 (segment (start 63.405978 81.68) (end 63.205489 81.479511) (width 0.25) (layer "F.Cu") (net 26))
 (segment (start 65.278 74.943) (end 67.26 74.943) (width 0.25) (layer "F.Cu") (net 26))
 (segment (start 68.595 74.993) (end 69.42 74.168) (width 0.25) (layer "F.Cu") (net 26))
 (segment (start 79.660511 72.919501) (end 78.972499 72.231489) (width 0.25) (layer "F.Cu") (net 26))
 (segment (start 79.660511 73.892499) (end 79.660511 72.919501) (width 0.25) (layer "F.Cu") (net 26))
 (segment (start 67.26 74.943) (end 67.31 74.993) (width 0.25) (layer "F.Cu") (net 26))
 (segment (start 63.205489 81.479511) (end 63.205489 77.015511) (width 0.25) (layer "F.Cu") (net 26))
 (segment (start 78.972499 72.231489) (end 71.356511 72.231489) (width 0.25) (layer "F.Cu") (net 26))
 (segment (start 62.16 82.48) (end 64.33 82.48) (width 0.25) (layer "F.Cu") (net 27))
 (segment (start 61.214 81.534) (end 62.16 82.48) (width 0.25) (layer "F.Cu") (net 27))
 (segment (start 61.214 84.074) (end 62.008 83.28) (width 0.25) (layer "F.Cu") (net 28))
 (segment (start 62.008 83.28) (end 64.33 83.28) (width 0.25) (layer "F.Cu") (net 28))
 (segment (start 80.455 82.126666) (end 78.0035 82.126666) (width 0.25) (layer "F.Cu") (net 30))
 (segment (start 80.455 78.74) (end 78.0035 78.74) (width 0.25) (layer "F.Cu") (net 33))
 (segment (start 78.0035 80.433333) (end 80.455 80.433333) (width 0.25) (layer "F.Cu") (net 5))
 (segment (start 78.0035 83.82) (end 80.455 83.82) (width 0.25) (layer "F.Cu") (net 7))
 (segment (start 61.214 78.11501) (end 62.388511 76.940499) (width 0.25) (layer "F.Cu") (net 31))
 (segment (start 62.388511 76.940499) (end 62.388511 75.279489) (width 0.25) (layer "F.Cu") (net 31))
 (segment (start 62.388511 75.279489) (end 64.275 73.393) (width 0.25) (layer "F.Cu") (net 31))
 (segment (start 64.275 73.393) (end 65.278 73.393) (width 0.25) (layer "F.Cu") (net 31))
 (segment (start 61.214 78.994) (end 61.214 78.11501) (width 0.25) (layer "F.Cu") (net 31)))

